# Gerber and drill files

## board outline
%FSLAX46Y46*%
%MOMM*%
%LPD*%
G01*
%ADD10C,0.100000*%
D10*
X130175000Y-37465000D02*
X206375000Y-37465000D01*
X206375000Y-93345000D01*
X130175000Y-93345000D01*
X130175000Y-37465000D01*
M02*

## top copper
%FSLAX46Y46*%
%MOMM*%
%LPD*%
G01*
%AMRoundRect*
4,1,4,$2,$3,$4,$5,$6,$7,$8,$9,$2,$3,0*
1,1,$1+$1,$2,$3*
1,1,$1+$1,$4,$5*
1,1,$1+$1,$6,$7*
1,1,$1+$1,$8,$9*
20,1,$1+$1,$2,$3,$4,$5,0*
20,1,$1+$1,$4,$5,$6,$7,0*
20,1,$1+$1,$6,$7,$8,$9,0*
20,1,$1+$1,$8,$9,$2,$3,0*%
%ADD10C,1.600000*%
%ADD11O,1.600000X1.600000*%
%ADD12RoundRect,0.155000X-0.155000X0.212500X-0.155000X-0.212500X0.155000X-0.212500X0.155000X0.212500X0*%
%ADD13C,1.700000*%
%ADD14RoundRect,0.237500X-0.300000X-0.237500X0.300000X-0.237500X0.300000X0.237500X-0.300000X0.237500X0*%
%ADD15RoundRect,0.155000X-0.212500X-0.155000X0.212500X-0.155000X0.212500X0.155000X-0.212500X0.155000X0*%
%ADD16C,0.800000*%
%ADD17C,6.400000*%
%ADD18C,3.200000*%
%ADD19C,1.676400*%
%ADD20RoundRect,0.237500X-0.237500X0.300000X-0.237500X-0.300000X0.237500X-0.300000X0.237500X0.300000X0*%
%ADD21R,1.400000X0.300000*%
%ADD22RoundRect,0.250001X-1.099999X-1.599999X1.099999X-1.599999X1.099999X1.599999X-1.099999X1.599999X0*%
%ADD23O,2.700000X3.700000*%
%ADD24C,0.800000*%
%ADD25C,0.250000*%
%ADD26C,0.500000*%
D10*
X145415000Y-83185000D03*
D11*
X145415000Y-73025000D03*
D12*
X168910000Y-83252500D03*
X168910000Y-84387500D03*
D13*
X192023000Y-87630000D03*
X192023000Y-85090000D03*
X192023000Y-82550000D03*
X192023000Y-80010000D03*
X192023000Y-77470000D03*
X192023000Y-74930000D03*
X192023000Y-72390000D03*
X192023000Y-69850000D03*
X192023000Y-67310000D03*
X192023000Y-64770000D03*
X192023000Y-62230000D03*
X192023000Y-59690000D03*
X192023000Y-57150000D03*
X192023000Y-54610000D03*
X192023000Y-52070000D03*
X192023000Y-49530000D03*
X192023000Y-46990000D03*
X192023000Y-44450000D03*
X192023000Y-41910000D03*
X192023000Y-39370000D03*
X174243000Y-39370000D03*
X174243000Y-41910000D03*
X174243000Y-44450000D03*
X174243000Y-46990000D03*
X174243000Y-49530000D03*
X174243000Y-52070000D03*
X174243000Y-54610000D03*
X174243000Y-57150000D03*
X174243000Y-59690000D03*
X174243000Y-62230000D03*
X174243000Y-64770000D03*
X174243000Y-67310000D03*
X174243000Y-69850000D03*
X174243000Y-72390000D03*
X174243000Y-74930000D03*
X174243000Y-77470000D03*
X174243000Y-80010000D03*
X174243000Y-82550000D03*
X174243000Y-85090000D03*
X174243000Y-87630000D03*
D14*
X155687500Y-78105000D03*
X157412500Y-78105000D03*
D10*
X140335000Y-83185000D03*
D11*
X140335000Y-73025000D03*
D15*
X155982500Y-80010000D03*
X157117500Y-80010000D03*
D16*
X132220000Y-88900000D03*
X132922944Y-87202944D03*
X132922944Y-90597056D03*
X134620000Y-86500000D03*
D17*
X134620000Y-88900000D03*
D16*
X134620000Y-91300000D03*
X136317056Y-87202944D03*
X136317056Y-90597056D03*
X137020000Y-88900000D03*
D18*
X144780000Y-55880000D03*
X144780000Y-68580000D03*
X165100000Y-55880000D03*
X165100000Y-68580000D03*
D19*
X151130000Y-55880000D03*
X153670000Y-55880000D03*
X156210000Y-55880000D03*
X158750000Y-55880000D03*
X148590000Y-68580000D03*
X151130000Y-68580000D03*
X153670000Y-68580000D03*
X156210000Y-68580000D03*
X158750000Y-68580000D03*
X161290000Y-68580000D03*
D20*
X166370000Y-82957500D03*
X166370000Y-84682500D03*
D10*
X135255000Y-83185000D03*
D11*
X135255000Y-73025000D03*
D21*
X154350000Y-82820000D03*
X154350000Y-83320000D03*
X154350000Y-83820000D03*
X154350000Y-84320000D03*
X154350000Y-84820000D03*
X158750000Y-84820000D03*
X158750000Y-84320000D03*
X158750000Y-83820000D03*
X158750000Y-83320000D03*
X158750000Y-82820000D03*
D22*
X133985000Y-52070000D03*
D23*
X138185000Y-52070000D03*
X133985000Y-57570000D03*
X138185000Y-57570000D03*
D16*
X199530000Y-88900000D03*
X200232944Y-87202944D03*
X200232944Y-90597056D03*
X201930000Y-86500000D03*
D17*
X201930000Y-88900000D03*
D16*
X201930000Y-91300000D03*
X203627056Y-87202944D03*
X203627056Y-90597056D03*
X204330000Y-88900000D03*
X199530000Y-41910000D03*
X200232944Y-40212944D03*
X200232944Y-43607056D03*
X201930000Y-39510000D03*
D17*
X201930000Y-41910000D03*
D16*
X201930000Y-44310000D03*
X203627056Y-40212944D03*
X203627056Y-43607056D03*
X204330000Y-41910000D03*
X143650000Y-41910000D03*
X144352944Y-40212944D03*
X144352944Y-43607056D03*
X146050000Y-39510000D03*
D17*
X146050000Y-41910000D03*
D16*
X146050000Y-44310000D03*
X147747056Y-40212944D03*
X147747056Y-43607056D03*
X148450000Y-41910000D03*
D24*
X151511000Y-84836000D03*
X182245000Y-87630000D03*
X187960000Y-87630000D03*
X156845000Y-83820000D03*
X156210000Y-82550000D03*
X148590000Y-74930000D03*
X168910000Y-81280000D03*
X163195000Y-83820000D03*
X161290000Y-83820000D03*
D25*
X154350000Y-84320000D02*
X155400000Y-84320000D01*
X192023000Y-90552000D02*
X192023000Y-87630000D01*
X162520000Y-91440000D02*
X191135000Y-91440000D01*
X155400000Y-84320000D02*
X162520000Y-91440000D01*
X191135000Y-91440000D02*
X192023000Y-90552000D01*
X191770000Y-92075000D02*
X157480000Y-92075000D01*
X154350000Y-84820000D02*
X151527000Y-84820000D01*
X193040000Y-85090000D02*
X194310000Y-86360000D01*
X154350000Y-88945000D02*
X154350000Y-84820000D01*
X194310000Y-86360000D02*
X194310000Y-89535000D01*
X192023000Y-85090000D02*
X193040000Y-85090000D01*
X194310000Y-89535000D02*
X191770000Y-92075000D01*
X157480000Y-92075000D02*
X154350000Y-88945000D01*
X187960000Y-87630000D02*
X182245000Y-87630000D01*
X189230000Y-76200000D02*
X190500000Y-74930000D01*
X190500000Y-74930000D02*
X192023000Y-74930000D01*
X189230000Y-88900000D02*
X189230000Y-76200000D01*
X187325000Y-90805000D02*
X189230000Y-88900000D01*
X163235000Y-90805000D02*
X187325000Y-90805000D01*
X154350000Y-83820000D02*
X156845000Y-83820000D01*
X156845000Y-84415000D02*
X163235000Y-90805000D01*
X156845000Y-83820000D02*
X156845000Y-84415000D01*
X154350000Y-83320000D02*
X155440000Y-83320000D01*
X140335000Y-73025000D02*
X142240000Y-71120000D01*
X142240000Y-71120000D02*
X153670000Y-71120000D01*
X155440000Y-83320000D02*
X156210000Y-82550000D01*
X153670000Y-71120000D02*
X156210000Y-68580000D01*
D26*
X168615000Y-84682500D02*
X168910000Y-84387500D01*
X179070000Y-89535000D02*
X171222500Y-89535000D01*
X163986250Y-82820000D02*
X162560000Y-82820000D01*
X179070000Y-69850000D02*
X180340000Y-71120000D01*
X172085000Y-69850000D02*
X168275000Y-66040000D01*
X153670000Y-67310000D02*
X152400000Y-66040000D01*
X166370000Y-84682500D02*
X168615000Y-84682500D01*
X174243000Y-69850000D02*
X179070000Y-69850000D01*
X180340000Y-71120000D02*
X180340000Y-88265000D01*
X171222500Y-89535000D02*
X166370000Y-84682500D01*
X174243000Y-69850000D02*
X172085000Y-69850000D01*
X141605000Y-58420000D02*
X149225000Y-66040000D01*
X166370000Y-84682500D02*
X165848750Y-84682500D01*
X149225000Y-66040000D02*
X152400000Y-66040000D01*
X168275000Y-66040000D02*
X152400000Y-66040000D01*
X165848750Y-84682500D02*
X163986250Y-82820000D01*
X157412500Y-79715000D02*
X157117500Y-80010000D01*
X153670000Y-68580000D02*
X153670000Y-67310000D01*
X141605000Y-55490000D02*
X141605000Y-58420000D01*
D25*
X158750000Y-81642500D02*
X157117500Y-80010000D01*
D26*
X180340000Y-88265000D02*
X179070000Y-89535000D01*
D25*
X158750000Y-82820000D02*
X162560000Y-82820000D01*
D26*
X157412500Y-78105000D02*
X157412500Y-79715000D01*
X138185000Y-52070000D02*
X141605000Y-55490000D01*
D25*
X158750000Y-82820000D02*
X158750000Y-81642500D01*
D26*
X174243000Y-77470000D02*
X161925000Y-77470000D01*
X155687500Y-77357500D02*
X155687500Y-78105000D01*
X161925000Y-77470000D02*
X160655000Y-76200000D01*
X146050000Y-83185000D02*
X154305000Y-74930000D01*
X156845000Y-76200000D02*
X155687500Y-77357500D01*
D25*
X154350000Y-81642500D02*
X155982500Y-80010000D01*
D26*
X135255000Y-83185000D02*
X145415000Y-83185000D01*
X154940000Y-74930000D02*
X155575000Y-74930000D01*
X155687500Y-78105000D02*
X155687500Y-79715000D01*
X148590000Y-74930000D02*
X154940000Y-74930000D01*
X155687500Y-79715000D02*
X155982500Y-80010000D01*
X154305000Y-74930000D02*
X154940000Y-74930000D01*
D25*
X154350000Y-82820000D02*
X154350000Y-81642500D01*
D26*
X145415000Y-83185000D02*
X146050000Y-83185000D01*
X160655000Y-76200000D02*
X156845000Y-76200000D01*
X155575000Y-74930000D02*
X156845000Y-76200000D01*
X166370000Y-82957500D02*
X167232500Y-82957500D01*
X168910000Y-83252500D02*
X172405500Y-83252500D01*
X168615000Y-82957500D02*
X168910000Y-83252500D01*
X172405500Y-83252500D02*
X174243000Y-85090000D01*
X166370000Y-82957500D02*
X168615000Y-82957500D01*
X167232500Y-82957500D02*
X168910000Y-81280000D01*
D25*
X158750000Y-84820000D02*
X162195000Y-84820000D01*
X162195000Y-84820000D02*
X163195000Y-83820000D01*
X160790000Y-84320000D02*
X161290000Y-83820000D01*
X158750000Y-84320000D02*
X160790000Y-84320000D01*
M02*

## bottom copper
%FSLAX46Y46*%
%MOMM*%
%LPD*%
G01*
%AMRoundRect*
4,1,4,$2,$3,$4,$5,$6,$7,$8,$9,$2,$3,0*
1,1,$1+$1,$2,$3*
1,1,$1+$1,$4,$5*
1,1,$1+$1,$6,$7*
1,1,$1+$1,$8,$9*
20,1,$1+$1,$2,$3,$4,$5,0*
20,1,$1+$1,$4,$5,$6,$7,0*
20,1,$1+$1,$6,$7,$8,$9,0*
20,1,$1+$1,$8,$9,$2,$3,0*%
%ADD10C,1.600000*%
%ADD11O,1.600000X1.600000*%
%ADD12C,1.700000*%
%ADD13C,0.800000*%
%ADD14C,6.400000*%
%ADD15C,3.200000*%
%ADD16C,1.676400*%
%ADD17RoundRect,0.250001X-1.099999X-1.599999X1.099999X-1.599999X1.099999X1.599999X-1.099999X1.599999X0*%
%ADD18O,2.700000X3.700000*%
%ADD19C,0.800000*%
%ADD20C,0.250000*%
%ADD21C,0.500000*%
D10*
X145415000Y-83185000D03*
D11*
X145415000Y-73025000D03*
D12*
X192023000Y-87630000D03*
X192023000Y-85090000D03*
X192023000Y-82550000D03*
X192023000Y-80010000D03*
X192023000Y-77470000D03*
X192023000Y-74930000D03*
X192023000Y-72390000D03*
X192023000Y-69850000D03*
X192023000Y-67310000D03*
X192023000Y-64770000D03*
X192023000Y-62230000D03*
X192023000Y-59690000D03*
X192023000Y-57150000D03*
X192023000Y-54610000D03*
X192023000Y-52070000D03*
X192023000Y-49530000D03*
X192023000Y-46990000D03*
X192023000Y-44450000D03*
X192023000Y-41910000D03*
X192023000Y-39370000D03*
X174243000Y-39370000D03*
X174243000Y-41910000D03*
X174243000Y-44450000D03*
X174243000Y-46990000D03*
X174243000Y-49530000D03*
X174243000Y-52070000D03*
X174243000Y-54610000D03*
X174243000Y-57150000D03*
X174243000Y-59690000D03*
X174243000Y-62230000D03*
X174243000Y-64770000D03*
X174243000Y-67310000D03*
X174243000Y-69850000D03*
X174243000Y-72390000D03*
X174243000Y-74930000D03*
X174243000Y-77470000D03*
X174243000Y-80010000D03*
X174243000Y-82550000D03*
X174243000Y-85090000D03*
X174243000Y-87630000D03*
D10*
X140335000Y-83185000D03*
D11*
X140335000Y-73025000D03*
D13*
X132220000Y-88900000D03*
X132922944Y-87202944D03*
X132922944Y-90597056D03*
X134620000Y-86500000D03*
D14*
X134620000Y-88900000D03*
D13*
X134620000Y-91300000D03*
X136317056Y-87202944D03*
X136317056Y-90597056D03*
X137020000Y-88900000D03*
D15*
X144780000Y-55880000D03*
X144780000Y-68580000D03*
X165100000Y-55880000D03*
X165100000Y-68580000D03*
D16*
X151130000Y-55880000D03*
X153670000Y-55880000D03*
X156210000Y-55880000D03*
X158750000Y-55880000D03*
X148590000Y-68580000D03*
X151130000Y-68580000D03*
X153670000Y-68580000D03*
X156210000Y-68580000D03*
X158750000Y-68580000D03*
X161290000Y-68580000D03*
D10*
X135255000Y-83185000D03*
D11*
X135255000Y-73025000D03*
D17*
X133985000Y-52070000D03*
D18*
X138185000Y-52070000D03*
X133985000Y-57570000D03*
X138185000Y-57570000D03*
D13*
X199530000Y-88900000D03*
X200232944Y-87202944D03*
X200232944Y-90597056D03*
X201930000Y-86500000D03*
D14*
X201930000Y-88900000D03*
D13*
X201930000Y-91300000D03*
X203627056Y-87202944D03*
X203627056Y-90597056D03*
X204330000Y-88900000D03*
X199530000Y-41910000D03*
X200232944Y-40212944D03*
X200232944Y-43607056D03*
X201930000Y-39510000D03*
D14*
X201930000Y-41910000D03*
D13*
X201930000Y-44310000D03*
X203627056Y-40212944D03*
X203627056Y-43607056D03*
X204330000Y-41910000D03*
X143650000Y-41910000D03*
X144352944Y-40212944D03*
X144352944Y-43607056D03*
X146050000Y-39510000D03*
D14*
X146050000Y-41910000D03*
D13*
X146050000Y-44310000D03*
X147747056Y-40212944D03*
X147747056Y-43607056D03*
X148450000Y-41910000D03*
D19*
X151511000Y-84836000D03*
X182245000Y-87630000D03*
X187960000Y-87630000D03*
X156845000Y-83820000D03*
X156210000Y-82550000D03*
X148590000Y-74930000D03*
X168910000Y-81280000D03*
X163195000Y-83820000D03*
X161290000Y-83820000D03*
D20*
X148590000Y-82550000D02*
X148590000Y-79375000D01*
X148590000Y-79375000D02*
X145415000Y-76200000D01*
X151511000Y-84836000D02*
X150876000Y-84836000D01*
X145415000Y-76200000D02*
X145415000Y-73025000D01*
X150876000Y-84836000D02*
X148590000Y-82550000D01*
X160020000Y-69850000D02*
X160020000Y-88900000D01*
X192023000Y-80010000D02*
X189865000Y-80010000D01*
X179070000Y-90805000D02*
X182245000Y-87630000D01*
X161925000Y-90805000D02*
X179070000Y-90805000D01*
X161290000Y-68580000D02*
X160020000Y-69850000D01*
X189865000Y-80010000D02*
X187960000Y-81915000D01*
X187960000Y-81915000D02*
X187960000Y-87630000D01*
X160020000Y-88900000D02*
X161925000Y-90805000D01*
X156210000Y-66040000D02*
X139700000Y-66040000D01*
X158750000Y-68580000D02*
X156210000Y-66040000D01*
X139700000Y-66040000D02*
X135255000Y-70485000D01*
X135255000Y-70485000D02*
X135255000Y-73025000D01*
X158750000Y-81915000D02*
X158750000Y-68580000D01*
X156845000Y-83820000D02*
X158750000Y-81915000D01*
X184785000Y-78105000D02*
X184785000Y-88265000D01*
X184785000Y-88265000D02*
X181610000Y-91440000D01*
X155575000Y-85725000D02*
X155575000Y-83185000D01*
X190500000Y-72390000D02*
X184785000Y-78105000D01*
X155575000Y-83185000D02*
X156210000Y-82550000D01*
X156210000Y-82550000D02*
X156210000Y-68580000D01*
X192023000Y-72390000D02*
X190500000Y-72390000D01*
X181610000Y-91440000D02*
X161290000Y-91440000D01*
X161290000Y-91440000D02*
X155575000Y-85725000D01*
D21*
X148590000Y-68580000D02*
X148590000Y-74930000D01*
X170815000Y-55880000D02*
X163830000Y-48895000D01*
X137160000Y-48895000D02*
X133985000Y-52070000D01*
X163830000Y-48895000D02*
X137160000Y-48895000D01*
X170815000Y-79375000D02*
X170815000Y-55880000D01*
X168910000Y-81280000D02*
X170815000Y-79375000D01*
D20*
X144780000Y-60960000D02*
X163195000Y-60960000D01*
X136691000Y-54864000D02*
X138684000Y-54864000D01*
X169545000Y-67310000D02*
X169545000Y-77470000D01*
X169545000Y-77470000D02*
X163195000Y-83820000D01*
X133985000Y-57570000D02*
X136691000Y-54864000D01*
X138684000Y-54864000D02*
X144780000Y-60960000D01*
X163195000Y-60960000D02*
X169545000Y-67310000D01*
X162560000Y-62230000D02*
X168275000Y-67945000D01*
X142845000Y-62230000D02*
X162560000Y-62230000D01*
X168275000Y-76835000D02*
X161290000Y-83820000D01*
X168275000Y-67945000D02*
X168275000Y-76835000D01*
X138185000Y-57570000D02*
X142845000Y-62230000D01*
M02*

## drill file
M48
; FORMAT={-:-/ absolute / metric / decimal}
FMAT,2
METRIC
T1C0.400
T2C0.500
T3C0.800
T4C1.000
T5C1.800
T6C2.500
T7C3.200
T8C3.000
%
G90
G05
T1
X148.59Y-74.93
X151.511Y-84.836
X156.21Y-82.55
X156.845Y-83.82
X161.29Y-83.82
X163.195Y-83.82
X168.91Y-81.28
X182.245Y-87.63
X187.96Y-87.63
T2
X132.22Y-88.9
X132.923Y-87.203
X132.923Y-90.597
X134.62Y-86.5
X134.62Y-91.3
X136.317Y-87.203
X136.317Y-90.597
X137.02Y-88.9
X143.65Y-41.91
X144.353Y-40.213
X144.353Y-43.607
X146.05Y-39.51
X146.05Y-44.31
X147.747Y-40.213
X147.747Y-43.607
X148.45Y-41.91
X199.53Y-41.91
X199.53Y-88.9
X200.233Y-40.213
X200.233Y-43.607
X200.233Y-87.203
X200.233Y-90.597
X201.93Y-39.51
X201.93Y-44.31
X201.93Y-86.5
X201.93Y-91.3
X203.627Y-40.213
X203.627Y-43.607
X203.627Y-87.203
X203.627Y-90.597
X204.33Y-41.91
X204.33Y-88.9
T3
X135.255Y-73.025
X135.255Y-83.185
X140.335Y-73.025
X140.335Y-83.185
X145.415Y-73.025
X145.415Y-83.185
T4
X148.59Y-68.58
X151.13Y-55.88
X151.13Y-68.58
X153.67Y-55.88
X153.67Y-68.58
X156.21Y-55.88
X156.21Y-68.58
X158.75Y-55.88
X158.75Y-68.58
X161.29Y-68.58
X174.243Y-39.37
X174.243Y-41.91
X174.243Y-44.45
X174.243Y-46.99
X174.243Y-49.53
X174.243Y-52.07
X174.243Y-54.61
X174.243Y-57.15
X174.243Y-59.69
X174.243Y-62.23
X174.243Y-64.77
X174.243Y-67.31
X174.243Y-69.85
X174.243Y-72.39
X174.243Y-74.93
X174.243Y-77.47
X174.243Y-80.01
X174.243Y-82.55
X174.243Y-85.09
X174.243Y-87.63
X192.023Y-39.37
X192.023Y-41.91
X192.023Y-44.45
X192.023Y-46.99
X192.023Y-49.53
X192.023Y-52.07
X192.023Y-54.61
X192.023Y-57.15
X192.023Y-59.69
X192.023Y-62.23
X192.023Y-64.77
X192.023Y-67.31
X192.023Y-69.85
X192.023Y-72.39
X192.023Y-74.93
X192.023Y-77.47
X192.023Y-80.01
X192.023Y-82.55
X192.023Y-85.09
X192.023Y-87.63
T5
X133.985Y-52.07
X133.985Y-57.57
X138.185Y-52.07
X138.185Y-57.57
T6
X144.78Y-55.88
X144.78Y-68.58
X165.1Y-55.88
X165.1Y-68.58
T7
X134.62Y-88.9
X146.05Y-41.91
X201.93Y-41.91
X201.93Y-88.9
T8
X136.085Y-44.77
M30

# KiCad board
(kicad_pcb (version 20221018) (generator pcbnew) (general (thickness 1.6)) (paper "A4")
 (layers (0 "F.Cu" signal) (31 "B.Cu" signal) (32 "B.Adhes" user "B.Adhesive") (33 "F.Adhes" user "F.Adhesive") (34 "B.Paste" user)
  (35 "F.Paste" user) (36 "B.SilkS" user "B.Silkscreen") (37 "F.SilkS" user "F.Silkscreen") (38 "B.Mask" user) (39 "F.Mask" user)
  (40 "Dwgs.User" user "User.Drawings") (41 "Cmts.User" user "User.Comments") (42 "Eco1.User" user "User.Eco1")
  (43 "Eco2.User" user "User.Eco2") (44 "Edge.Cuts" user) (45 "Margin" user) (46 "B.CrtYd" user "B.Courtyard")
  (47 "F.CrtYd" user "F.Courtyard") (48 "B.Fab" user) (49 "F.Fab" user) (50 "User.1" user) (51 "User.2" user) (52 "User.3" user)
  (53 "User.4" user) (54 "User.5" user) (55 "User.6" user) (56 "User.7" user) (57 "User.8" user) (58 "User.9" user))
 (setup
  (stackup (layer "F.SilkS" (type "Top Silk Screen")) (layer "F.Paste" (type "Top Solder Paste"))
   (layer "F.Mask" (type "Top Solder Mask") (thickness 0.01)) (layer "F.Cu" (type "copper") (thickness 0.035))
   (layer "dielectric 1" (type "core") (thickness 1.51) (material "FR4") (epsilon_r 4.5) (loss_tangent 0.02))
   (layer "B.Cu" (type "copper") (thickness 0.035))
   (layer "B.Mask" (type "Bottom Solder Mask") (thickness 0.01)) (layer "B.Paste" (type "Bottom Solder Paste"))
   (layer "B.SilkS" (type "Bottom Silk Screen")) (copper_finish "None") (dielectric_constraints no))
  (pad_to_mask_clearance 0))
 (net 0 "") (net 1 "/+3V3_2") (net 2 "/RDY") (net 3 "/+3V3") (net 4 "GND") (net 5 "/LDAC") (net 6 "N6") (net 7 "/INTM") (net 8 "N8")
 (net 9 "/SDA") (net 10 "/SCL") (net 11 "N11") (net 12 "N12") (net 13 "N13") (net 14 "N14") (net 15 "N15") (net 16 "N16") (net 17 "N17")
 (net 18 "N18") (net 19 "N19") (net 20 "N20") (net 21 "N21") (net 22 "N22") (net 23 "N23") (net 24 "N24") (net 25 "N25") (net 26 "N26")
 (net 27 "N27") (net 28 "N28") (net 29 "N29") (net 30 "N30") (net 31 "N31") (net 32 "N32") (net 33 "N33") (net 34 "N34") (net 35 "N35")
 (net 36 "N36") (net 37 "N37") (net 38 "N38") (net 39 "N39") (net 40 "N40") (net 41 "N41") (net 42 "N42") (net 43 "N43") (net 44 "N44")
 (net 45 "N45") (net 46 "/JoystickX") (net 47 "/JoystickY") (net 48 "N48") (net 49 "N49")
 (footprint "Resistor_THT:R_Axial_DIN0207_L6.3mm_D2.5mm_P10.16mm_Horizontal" (layer "F.Cu") (at 145.415 83.185 90)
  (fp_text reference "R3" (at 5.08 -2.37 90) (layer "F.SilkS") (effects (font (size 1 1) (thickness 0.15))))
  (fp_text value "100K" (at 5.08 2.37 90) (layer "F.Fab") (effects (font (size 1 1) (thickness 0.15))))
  (pad "1" thru_hole circle (at 0 0 90) (size 1.6 1.6) (drill 0.8) (layers "*.Cu" "*.Mask") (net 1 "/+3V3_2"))
  (pad "2" thru_hole oval (at 10.16 0 90) (size 1.6 1.6) (drill 0.8) (layers "*.Cu" "*.Mask") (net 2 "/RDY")))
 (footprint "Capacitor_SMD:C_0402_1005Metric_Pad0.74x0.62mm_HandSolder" (layer "F.Cu") (at 168.91 83.82 -90)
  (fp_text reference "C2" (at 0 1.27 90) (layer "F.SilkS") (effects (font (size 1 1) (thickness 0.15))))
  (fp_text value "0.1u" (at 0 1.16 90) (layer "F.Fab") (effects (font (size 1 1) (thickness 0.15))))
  (pad "1" smd roundrect (at -0.5675 0 270) (size 0.735 0.62) (layers "F.Cu" "F.Paste" "F.Mask") (roundrect_rratio 0.25) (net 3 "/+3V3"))
  (pad "2" smd roundrect (at 0.5675 0 270) (size 0.735 0.62) (layers "F.Cu" "F.Paste" "F.Mask") (roundrect_rratio 0.25) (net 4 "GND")))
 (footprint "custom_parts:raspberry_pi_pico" (layer "F.Cu") (at 183.515 64.712 90)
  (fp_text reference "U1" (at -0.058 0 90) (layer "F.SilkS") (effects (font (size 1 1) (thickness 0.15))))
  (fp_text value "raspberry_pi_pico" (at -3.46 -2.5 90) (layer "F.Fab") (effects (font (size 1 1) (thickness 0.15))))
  (pad "1" thru_hole circle (at -22.918 8.508) (size 1.7 1.7) (drill 1) (layers "*.Cu" "*.Mask") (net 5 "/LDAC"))
  (pad "2" thru_hole circle (at -20.378 8.508) (size 1.7 1.7) (drill 1) (layers "*.Cu" "*.Mask") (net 2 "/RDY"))
  (pad "3" thru_hole circle (at -17.838 8.508) (size 1.7 1.7) (drill 1) (layers "*.Cu" "*.Mask") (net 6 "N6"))
  (pad "4" thru_hole circle (at -15.298 8.508) (size 1.7 1.7) (drill 1) (layers "*.Cu" "*.Mask") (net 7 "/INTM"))
  (pad "5" thru_hole circle (at -12.758 8.508) (size 1.7 1.7) (drill 1) (layers "*.Cu" "*.Mask") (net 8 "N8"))
  (pad "6" thru_hole circle (at -10.218 8.508) (size 1.7 1.7) (drill 1) (layers "*.Cu" "*.Mask") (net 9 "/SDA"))
  (pad "7" thru_hole circle (at -7.678 8.508) (size 1.7 1.7) (drill 1) (layers "*.Cu" "*.Mask") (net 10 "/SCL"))
  (pad "8" thru_hole circle (at -5.138 8.508) (size 1.7 1.7) (drill 1) (layers "*.Cu" "*.Mask") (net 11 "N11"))
  (pad "9" thru_hole circle (at -2.598 8.508) (size 1.7 1.7) (drill 1) (layers "*.Cu" "*.Mask") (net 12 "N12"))
  (pad "10" thru_hole circle (at -0.058 8.508) (size 1.7 1.7) (drill 1) (layers "*.Cu" "*.Mask") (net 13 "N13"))
  (pad "11" thru_hole circle (at 2.482 8.508) (size 1.7 1.7) (drill 1) (layers "*.Cu" "*.Mask") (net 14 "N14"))
  (pad "12" thru_hole circle (at 5.022 8.508) (size 1.7 1.7) (drill 1) (layers "*.Cu" "*.Mask") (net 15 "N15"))
  (pad "13" thru_hole circle (at 7.562 8.508) (size 1.7 1.7) (drill 1) (layers "*.Cu" "*.Mask") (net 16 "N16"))
  (pad "14" thru_hole circle (at 10.102 8.508) (size 1.7 1.7) (drill 1) (layers "*.Cu" "*.Mask") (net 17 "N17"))
  (pad "15" thru_hole circle (at 12.642 8.508) (size 1.7 1.7) (drill 1) (layers "*.Cu" "*.Mask") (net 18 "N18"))
  (pad "16" thru_hole circle (at 15.182 8.508) (size 1.7 1.7) (drill 1) (layers "*.Cu" "*.Mask") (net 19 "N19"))
  (pad "17" thru_hole circle (at 17.722 8.508) (size 1.7 1.7) (drill 1) (layers "*.Cu" "*.Mask") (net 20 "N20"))
  (pad "18" thru_hole circle (at 20.262 8.508) (size 1.7 1.7) (drill 1) (layers "*.Cu" "*.Mask") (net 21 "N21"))
  (pad "19" thru_hole circle (at 22.802 8.508) (size 1.7 1.7) (drill 1) (layers "*.Cu" "*.Mask") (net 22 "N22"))
  (pad "20" thru_hole circle (at 25.342 8.508) (size 1.7 1.7) (drill 1) (layers "*.Cu" "*.Mask") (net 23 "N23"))
  (pad "21" thru_hole circle (at 25.342 -9.272) (size 1.7 1.7) (drill 1) (layers "*.Cu" "*.Mask") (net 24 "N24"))
  (pad "22" thru_hole circle (at 22.802 -9.272) (size 1.7 1.7) (drill 1) (layers "*.Cu" "*.Mask") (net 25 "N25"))
  (pad "23" thru_hole circle (at 20.262 -9.272) (size 1.7 1.7) (drill 1) (layers "*.Cu" "*.Mask") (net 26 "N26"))
  (pad "24" thru_hole circle (at 17.722 -9.272) (size 1.7 1.7) (drill 1) (layers "*.Cu" "*.Mask") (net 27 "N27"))
  (pad "25" thru_hole circle (at 15.182 -9.272) (size 1.7 1.7) (drill 1) (layers "*.Cu" "*.Mask") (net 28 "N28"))
  (pad "26" thru_hole circle (at 12.642 -9.272) (size 1.7 1.7) (drill 1) (layers "*.Cu" "*.Mask") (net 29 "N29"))
  (pad "27" thru_hole circle (at 10.102 -9.272) (size 1.7 1.7) (drill 1) (layers "*.Cu" "*.Mask") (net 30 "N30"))
  (pad "28" thru_hole circle (at 7.562 -9.272) (size 1.7 1.7) (drill 1) (layers "*.Cu" "*.Mask") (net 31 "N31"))
  (pad "29" thru_hole circle (at 5.022 -9.272) (size 1.7 1.7) (drill 1) (layers "*.Cu" "*.Mask") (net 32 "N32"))
  (pad "30" thru_hole circle (at 2.482 -9.272) (size 1.7 1.7) (drill 1) (layers "*.Cu" "*.Mask") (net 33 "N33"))
  (pad "31" thru_hole circle (at -0.058 -9.272) (size 1.7 1.7) (drill 1) (layers "*.Cu" "*.Mask") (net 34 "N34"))
  (pad "32" thru_hole circle (at -2.598 -9.272) (size 1.7 1.7) (drill 1) (layers "*.Cu" "*.Mask") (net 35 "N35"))
  (pad "33" thru_hole circle (at -5.138 -9.272) (size 1.7 1.7) (drill 1) (layers "*.Cu" "*.Mask") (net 4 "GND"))
  (pad "34" thru_hole circle (at -7.678 -9.272) (size 1.7 1.7) (drill 1) (layers "*.Cu" "*.Mask") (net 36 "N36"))
  (pad "35" thru_hole circle (at -10.218 -9.272) (size 1.7 1.7) (drill 1) (layers "*.Cu" "*.Mask") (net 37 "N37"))
  (pad "36" thru_hole circle (at -12.758 -9.272) (size 1.7 1.7) (drill 1) (layers "*.Cu" "*.Mask") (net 1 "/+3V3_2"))
  (pad "37" thru_hole circle (at -15.298 -9.272) (size 1.7 1.7) (drill 1) (layers "*.Cu" "*.Mask") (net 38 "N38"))
  (pad "38" thru_hole circle (at -17.838 -9.272) (size 1.7 1.7) (drill 1) (layers "*.Cu" "*.Mask") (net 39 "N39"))
  (pad "39" thru_hole circle (at -20.378 -9.272) (size 1.7 1.7) (drill 1) (layers "*.Cu" "*.Mask") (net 3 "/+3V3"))
  (pad "40" thru_hole circle (at -22.918 -9.272) (size 1.7 1.7) (drill 1) (layers "*.Cu" "*.Mask") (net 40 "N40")))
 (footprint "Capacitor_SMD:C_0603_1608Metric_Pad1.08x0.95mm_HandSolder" (layer "F.Cu") (at 156.55 78.105)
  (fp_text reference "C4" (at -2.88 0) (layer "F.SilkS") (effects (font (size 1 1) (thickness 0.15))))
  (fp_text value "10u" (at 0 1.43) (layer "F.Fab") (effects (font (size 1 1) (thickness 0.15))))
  (pad "1" smd roundrect (at -0.8625 0) (size 1.075 0.95) (layers "F.Cu" "F.Paste" "F.Mask") (roundrect_rratio 0.25) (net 1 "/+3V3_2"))
  (pad "2" smd roundrect (at 0.8625 0) (size 1.075 0.95) (layers "F.Cu" "F.Paste" "F.Mask") (roundrect_rratio 0.25) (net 4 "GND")))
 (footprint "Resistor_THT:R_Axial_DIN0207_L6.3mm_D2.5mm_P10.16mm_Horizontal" (layer "F.Cu") (at 140.335 83.185 90)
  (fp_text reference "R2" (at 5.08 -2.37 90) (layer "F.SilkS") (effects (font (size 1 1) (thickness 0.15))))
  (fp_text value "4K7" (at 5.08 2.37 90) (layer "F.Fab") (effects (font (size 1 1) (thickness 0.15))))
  (pad "1" thru_hole circle (at 0 0 90) (size 1.6 1.6) (drill 0.8) (layers "*.Cu" "*.Mask") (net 1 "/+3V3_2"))
  (pad "2" thru_hole oval (at 10.16 0 90) (size 1.6 1.6) (drill 0.8) (layers "*.Cu" "*.Mask") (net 10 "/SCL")))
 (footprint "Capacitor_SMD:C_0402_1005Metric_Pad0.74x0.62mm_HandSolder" (layer "F.Cu") (at 156.55 80.01)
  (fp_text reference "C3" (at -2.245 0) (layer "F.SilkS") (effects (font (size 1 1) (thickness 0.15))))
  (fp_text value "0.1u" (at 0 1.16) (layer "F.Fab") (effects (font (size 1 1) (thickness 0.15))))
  (pad "1" smd roundrect (at -0.5675 0) (size 0.735 0.62) (layers "F.Cu" "F.Paste" "F.Mask") (roundrect_rratio 0.25) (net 1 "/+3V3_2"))
  (pad "2" smd roundrect (at 0.5675 0) (size 0.735 0.62) (layers "F.Cu" "F.Paste" "F.Mask") (roundrect_rratio 0.25) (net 4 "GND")))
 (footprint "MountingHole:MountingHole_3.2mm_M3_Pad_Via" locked (layer "F.Cu") (at 134.62 88.9)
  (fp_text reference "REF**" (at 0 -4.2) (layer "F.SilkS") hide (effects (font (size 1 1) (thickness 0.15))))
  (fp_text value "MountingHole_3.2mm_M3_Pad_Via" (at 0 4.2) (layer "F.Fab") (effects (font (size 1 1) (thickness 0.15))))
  (pad "1" thru_hole circle locked (at -2.4 0) (size 0.8 0.8) (drill 0.5) (layers "*.Cu" "*.Mask"))
  (pad "1" thru_hole circle locked (at -1.697056 -1.697056) (size 0.8 0.8) (drill 0.5) (layers "*.Cu" "*.Mask"))
  (pad "1" thru_hole circle locked (at -1.697056 1.697056) (size 0.8 0.8) (drill 0.5) (layers "*.Cu" "*.Mask"))
  (pad "1" thru_hole circle locked (at 0 -2.4) (size 0.8 0.8) (drill 0.5) (layers "*.Cu" "*.Mask"))
  (pad "1" thru_hole circle locked (at 0 0) (size 6.4 6.4) (drill 3.2) (layers "*.Cu" "*.Mask"))
  (pad "1" thru_hole circle locked (at 0 2.4) (size 0.8 0.8) (drill 0.5) (layers "*.Cu" "*.Mask"))
  (pad "1" thru_hole circle locked (at 1.697056 -1.697056) (size 0.8 0.8) (drill 0.5) (layers "*.Cu" "*.Mask"))
  (pad "1" thru_hole circle locked (at 1.697056 1.697056) (size 0.8 0.8) (drill 0.5) (layers "*.Cu" "*.Mask"))
  (pad "1" thru_hole circle locked (at 2.4 0) (size 0.8 0.8) (drill 0.5) (layers "*.Cu" "*.Mask")))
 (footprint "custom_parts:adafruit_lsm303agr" (layer "F.Cu") (at 154.94 63.5)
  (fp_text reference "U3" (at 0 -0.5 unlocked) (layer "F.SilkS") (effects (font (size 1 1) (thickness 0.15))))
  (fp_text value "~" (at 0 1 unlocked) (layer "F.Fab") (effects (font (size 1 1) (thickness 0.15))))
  (pad "" thru_hole circle (at -10.16 -7.62) (size 3.2 3.2) (drill 2.5) (layers "*.Cu" "*.Mask") (zone_connect 0))
  (pad "" thru_hole circle (at -10.16 5.08) (size 3.2 3.2) (drill 2.5) (layers "*.Cu" "*.Mask") (zone_connect 0))
  (pad "" thru_hole circle (at 10.16 -7.62) (size 3.2 3.2) (drill 2.5) (layers "*.Cu" "*.Mask") (zone_connect 0))
  (pad "" thru_hole circle (at 10.16 5.08) (size 3.2 3.2) (drill 2.5) (layers "*.Cu" "*.Mask") (zone_connect 0))
  (pad "0" thru_hole circle (at -3.81 -7.62 90) (size 1.6764 1.6764) (drill 1) (layers "*.Cu" "*.Mask") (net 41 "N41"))
  (pad "1" thru_hole circle (at -1.27 -7.62 90) (size 1.6764 1.6764) (drill 1) (layers "*.Cu" "*.Mask") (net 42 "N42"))
  (pad "2" thru_hole circle (at 1.27 -7.62 90) (size 1.6764 1.6764) (drill 1) (layers "*.Cu" "*.Mask") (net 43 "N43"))
  (pad "3" thru_hole circle (at 3.81 -7.62 90) (size 1.6764 1.6764) (drill 1) (layers "*.Cu" "*.Mask") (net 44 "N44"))
  (pad "4" thru_hole circle (at -6.35 5.08 90) (size 1.6764 1.6764) (drill 1) (layers "*.Cu" "*.Mask") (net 1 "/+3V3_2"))
  (pad "5" thru_hole circle (at -3.81 5.08 90) (size 1.6764 1.6764) (drill 1) (layers "*.Cu" "*.Mask") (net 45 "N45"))
  (pad "6" thru_hole circle (at -1.27 5.08 90) (size 1.6764 1.6764) (drill 1) (layers "*.Cu" "*.Mask") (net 4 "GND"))
  (pad "7" thru_hole circle (at 1.27 5.08 90) (size 1.6764 1.6764) (drill 1) (layers "*.Cu" "*.Mask") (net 10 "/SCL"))
  (pad "8" thru_hole circle (at 3.81 5.08 90) (size 1.6764 1.6764) (drill 1) (layers "*.Cu" "*.Mask") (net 9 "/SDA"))
  (pad "9" thru_hole circle (at 6.35 5.08 90) (size 1.6764 1.6764) (drill 1) (layers "*.Cu" "*.Mask") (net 7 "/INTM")))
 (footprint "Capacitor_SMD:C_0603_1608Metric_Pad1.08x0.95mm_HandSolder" (layer "F.Cu") (at 166.37 83.82 -90)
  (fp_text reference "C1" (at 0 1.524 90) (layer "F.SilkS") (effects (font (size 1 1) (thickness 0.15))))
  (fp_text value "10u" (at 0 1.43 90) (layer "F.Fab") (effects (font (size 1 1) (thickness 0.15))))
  (pad "1" smd roundrect (at -0.8625 0 270) (size 1.075 0.95) (layers "F.Cu" "F.Paste" "F.Mask") (roundrect_rratio 0.25) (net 3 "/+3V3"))
  (pad "2" smd roundrect (at 0.8625 0 270) (size 1.075 0.95) (layers "F.Cu" "F.Paste" "F.Mask") (roundrect_rratio 0.25) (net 4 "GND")))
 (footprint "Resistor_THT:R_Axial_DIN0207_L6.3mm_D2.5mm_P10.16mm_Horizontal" (layer "F.Cu") (at 135.255 83.185 90)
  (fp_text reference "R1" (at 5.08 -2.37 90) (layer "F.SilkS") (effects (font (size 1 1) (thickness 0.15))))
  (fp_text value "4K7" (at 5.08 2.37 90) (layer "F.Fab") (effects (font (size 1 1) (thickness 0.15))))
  (pad "1" thru_hole circle (at 0 0 90) (size 1.6 1.6) (drill 0.8) (layers "*.Cu" "*.Mask") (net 1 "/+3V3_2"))
  (pad "2" thru_hole oval (at 10.16 0 90) (size 1.6 1.6) (drill 0.8) (layers "*.Cu" "*.Mask") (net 9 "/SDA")))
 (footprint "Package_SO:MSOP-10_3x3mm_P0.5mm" (layer "F.Cu") (at 156.55 83.82)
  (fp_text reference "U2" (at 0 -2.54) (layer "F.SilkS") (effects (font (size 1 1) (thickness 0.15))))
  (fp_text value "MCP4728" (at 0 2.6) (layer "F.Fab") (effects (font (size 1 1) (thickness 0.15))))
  (pad "1" smd rect (at -2.2 -1) (size 1.4 0.3) (layers "F.Cu" "F.Paste" "F.Mask") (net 1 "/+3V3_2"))
  (pad "2" smd rect (at -2.2 -0.5) (size 1.4 0.3) (layers "F.Cu" "F.Paste" "F.Mask") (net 10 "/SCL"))
  (pad "3" smd rect (at -2.2 0) (size 1.4 0.3) (layers "F.Cu" "F.Paste" "F.Mask") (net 9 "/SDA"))
  (pad "4" smd rect (at -2.2 0.5) (size 1.4 0.3) (layers "F.Cu" "F.Paste" "F.Mask") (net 5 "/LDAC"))
  (pad "5" smd rect (at -2.2 1) (size 1.4 0.3) (layers "F.Cu" "F.Paste" "F.Mask") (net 2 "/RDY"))
  (pad "6" smd rect (at 2.2 1) (size 1.4 0.3) (layers "F.Cu" "F.Paste" "F.Mask") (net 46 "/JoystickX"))
  (pad "7" smd rect (at 2.2 0.5) (size 1.4 0.3) (layers "F.Cu" "F.Paste" "F.Mask") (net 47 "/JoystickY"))
  (pad "8" smd rect (at 2.2 0) (size 1.4 0.3) (layers "F.Cu" "F.Paste" "F.Mask") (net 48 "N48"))
  (pad "9" smd rect (at 2.2 -0.5) (size 1.4 0.3) (layers "F.Cu" "F.Paste" "F.Mask") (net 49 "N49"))
  (pad "10" smd rect (at 2.2 -1) (size 1.4 0.3) (layers "F.Cu" "F.Paste" "F.Mask") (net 4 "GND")))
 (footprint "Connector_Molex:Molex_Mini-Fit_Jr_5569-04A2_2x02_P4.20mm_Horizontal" (layer "F.Cu") (at 133.985 52.07)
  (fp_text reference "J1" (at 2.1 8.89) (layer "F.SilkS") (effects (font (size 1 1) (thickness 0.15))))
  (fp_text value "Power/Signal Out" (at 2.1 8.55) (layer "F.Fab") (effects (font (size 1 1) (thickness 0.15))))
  (pad "" np_thru_hole circle (at 2.1 -7.3) (size 3 3) (drill 3) (layers "*.Cu" "*.Mask"))
  (pad "1" thru_hole roundrect (at 0 0) (size 2.7 3.7) (drill 1.8) (layers "*.Cu" "*.Mask") (roundrect_rratio 0.09259296296) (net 3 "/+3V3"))
  (pad "2" thru_hole oval (at 4.2 0) (size 2.7 3.7) (drill 1.8) (layers "*.Cu" "*.Mask") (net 4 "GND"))
  (pad "3" thru_hole oval (at 0 5.5) (size 2.7 3.7) (drill 1.8) (layers "*.Cu" "*.Mask") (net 46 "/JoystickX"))
  (pad "4" thru_hole oval (at 4.2 5.5) (size 2.7 3.7) (drill 1.8) (layers "*.Cu" "*.Mask") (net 47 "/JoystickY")))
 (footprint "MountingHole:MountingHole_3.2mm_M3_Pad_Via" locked (layer "F.Cu") (at 201.93 88.9)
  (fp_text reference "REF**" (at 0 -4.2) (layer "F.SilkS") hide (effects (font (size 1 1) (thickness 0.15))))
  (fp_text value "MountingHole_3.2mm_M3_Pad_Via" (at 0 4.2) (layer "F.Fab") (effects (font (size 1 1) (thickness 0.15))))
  (pad "1" thru_hole circle locked (at -2.4 0) (size 0.8 0.8) (drill 0.5) (layers "*.Cu" "*.Mask"))
  (pad "1" thru_hole circle locked (at -1.697056 -1.697056) (size 0.8 0.8) (drill 0.5) (layers "*.Cu" "*.Mask"))
  (pad "1" thru_hole circle locked (at -1.697056 1.697056) (size 0.8 0.8) (drill 0.5) (layers "*.Cu" "*.Mask"))
  (pad "1" thru_hole circle locked (at 0 -2.4) (size 0.8 0.8) (drill 0.5) (layers "*.Cu" "*.Mask"))
  (pad "1" thru_hole circle locked (at 0 0) (size 6.4 6.4) (drill 3.2) (layers "*.Cu" "*.Mask"))
  (pad "1" thru_hole circle locked (at 0 2.4) (size 0.8 0.8) (drill 0.5) (layers "*.Cu" "*.Mask"))
  (pad "1" thru_hole circle locked (at 1.697056 -1.697056) (size 0.8 0.8) (drill 0.5) (layers "*.Cu" "*.Mask"))
  (pad "1" thru_hole circle locked (at 1.697056 1.697056) (size 0.8 0.8) (drill 0.5) (layers "*.Cu" "*.Mask"))
  (pad "1" thru_hole circle locked (at 2.4 0) (size 0.8 0.8) (drill 0.5) (layers "*.Cu" "*.Mask")))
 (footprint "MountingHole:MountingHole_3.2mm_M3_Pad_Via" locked (layer "F.Cu") (at 201.93 41.91)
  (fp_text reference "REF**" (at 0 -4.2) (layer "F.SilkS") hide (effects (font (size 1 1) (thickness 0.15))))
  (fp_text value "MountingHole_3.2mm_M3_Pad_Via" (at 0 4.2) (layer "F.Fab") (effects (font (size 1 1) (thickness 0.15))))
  (pad "1" thru_hole circle locked (at -2.4 0) (size 0.8 0.8) (drill 0.5) (layers "*.Cu" "*.Mask"))
  (pad "1" thru_hole circle locked (at -1.697056 -1.697056) (size 0.8 0.8) (drill 0.5) (layers "*.Cu" "*.Mask"))
  (pad "1" thru_hole circle locked (at -1.697056 1.697056) (size 0.8 0.8) (drill 0.5) (layers "*.Cu" "*.Mask"))
  (pad "1" thru_hole circle locked (at 0 -2.4) (size 0.8 0.8) (drill 0.5) (layers "*.Cu" "*.Mask"))
  (pad "1" thru_hole circle locked (at 0 0) (size 6.4 6.4) (drill 3.2) (layers "*.Cu" "*.Mask"))
  (pad "1" thru_hole circle locked (at 0 2.4) (size 0.8 0.8) (drill 0.5) (layers "*.Cu" "*.Mask"))
  (pad "1" thru_hole circle locked (at 1.697056 -1.697056) (size 0.8 0.8) (drill 0.5) (layers "*.Cu" "*.Mask"))
  (pad "1" thru_hole circle locked (at 1.697056 1.697056) (size 0.8 0.8) (drill 0.5) (layers "*.Cu" "*.Mask"))
  (pad "1" thru_hole circle locked (at 2.4 0) (size 0.8 0.8) (drill 0.5) (layers "*.Cu" "*.Mask")))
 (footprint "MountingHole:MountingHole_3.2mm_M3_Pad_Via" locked (layer "F.Cu") (at 146.05 41.91)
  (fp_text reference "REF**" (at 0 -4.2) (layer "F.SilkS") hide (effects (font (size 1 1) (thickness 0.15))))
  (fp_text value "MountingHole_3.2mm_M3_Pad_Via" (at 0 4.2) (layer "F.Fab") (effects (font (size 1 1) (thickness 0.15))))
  (pad "1" thru_hole circle locked (at -2.4 0) (size 0.8 0.8) (drill 0.5) (layers "*.Cu" "*.Mask"))
  (pad "1" thru_hole circle locked (at -1.697056 -1.697056) (size 0.8 0.8) (drill 0.5) (layers "*.Cu" "*.Mask"))
  (pad "1" thru_hole circle locked (at -1.697056 1.697056) (size 0.8 0.8) (drill 0.5) (layers "*.Cu" "*.Mask"))
  (pad "1" thru_hole circle locked (at 0 -2.4) (size 0.8 0.8) (drill 0.5) (layers "*.Cu" "*.Mask"))
  (pad "1" thru_hole circle locked (at 0 0) (size 6.4 6.4) (drill 3.2) (layers "*.Cu" "*.Mask"))
  (pad "1" thru_hole circle locked (at 0 2.4) (size 0.8 0.8) (drill 0.5) (layers "*.Cu" "*.Mask"))
  (pad "1" thru_hole circle locked (at 1.697056 -1.697056) (size 0.8 0.8) (drill 0.5) (layers "*.Cu" "*.Mask"))
  (pad "1" thru_hole circle locked (at 1.697056 1.697056) (size 0.8 0.8) (drill 0.5) (layers "*.Cu" "*.Mask"))
  (pad "1" thru_hole circle locked (at 2.4 0) (size 0.8 0.8) (drill 0.5) (layers "*.Cu" "*.Mask")))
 (gr_rect (start 130.175 37.465) (end 206.375 93.345) (stroke (width 0.1) (type default)) (fill none) (layer "Edge.Cuts"))
 (segment (start 154.35 84.32) (end 155.4 84.32) (width 0.25) (layer "F.Cu") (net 5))
 (segment (start 192.023 90.552) (end 192.023 87.63) (width 0.25) (layer "F.Cu") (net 5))
 (segment (start 162.52 91.44) (end 191.135 91.44) (width 0.25) (layer "F.Cu") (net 5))
 (segment (start 155.4 84.32) (end 162.52 91.44) (width 0.25) (layer "F.Cu") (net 5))
 (segment (start 191.135 91.44) (end 192.023 90.552) (width 0.25) (layer "F.Cu") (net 5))
 (segment (start 191.77 92.075) (end 157.48 92.075) (width 0.25) (layer "F.Cu") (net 2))
 (segment (start 154.35 84.82) (end 151.527 84.82) (width 0.25) (layer "F.Cu") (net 2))
 (segment (start 193.04 85.09) (end 194.31 86.36) (width 0.25) (layer "F.Cu") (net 2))
 (segment (start 154.35 88.945) (end 154.35 84.82) (width 0.25) (layer "F.Cu") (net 2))
 (segment (start 194.31 86.36) (end 194.31 89.535) (width 0.25) (layer "F.Cu") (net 2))
 (segment (start 192.023 85.09) (end 193.04 85.09) (width 0.25) (layer "F.Cu") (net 2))
 (segment (start 194.31 89.535) (end 191.77 92.075) (width 0.25) (layer "F.Cu") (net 2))
 (segment (start 157.48 92.075) (end 154.35 88.945) (width 0.25) (layer "F.Cu") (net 2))
 (via (at 151.511 84.836) (size 0.8) (drill 0.4) (layers "F.Cu" "B.Cu") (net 2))
 (segment (start 148.59 82.55) (end 148.59 79.375) (width 0.25) (layer "B.Cu") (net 2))
 (segment (start 148.59 79.375) (end 145.415 76.2) (width 0.25) (layer "B.Cu") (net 2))
 (segment (start 151.511 84.836) (end 150.876 84.836) (width 0.25) (layer "B.Cu") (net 2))
 (segment (start 145.415 76.2) (end 145.415 73.025) (width 0.25) (layer "B.Cu") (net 2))
 (segment (start 150.876 84.836) (end 148.59 82.55) (width 0.25) (layer "B.Cu") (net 2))
 (segment (start 187.96 87.63) (end 182.245 87.63) (width 0.25) (layer "F.Cu") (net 7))
 (via (at 182.245 87.63) (size 0.8) (drill 0.4) (layers "F.Cu" "B.Cu") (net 7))
 (via (at 187.96 87.63) (size 0.8) (drill 0.4) (layers "F.Cu" "B.Cu") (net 7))
 (segment (start 160.02 69.85) (end 160.02 88.9) (width 0.25) (layer "B.Cu") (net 7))
 (segment (start 192.023 80.01) (end 189.865 80.01) (width 0.25) (layer "B.Cu") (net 7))
 (segment (start 179.07 90.805) (end 182.245 87.63) (width 0.25) (layer "B.Cu") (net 7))
 (segment (start 161.925 90.805) (end 179.07 90.805) (width 0.25) (layer "B.Cu") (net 7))
 (segment (start 161.29 68.58) (end 160.02 69.85) (width 0.25) (layer "B.Cu") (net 7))
 (segment (start 189.865 80.01) (end 187.96 81.915) (width 0.25) (layer "B.Cu") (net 7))
 (segment (start 187.96 81.915) (end 187.96 87.63) (width 0.25) (layer "B.Cu") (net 7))
 (segment (start 160.02 88.9) (end 161.925 90.805) (width 0.25) (layer "B.Cu") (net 7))
 (segment (start 189.23 76.2) (end 190.5 74.93) (width 0.25) (layer "F.Cu") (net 9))
 (segment (start 190.5 74.93) (end 192.023 74.93) (width 0.25) (layer "F.Cu") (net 9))
 (segment (start 189.23 88.9) (end 189.23 76.2) (width 0.25) (layer "F.Cu") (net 9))
 (segment (start 187.325 90.805) (end 189.23 88.9) (width 0.25) (layer "F.Cu") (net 9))
 (segment (start 163.235 90.805) (end 187.325 90.805) (width 0.25) (layer "F.Cu") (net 9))
 (segment (start 154.35 83.82) (end 156.845 83.82) (width 0.25) (layer "F.Cu") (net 9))
 (segment (start 156.845 84.415) (end 163.235 90.805) (width 0.25) (layer "F.Cu") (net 9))
 (segment (start 156.845 83.82) (end 156.845 84.415) (width 0.25) (layer "F.Cu") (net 9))
 (via (at 156.845 83.82) (size 0.8) (drill 0.4) (layers "F.Cu" "B.Cu") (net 9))
 (segment (start 156.21 66.04) (end 139.7 66.04) (width 0.25) (layer "B.Cu") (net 9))
 (segment (start 158.75 68.58) (end 156.21 66.04) (width 0.25) (layer "B.Cu") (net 9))
 (segment (start 139.7 66.04) (end 135.255 70.485) (width 0.25) (layer "B.Cu") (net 9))
 (segment (start 135.255 70.485) (end 135.255 73.025) (width 0.25) (layer "B.Cu") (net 9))
 (segment (start 158.75 81.915) (end 158.75 68.58) (width 0.25) (layer "B.Cu") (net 9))
 (segment (start 156.845 83.82) (end 158.75 81.915) (width 0.25) (layer "B.Cu") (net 9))
 (segment (start 154.35 83.32) (end 155.44 83.32) (width 0.25) (layer "F.Cu") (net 10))
 (segment (start 140.335 73.025) (end 142.24 71.12) (width 0.25) (layer "F.Cu") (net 10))
 (segment (start 142.24 71.12) (end 153.67 71.12) (width 0.25) (layer "F.Cu") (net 10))
 (segment (start 155.44 83.32) (end 156.21 82.55) (width 0.25) (layer "F.Cu") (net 10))
 (segment (start 153.67 71.12) (end 156.21 68.58) (width 0.25) (layer "F.Cu") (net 10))
 (via (at 156.21 82.55) (size 0.8) (drill 0.4) (layers "F.Cu" "B.Cu") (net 10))
 (segment (start 184.785 78.105) (end 184.785 88.265) (width 0.25) (layer "B.Cu") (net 10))
 (segment (start 184.785 88.265) (end 181.61 91.44) (width 0.25) (layer "B.Cu") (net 10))
 (segment (start 155.575 85.725) (end 155.575 83.185) (width 0.25) (layer "B.Cu") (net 10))
 (segment (start 190.5 72.39) (end 184.785 78.105) (width 0.25) (layer "B.Cu") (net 10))
 (segment (start 155.575 83.185) (end 156.21 82.55) (width 0.25) (layer "B.Cu") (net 10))
 (segment (start 156.21 82.55) (end 156.21 68.58) (width 0.25) (layer "B.Cu") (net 10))
 (segment (start 192.023 72.39) (end 190.5 72.39) (width 0.25) (layer "B.Cu") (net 10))
 (segment (start 181.61 91.44) (end 161.29 91.44) (width 0.25) (layer "B.Cu") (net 10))
 (segment (start 161.29 91.44) (end 155.575 85.725) (width 0.25) (layer "B.Cu") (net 10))
 (segment (start 168.615 84.6825) (end 168.91 84.3875) (width 0.5) (layer "F.Cu") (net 4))
 (segment (start 179.07 89.535) (end 171.2225 89.535) (width 0.5) (layer "F.Cu") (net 4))
 (segment (start 163.98625 82.82) (end 162.56 82.82) (width 0.5) (layer "F.Cu") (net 4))
 (segment (start 179.07 69.85) (end 180.34 71.12) (width 0.5) (layer "F.Cu") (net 4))
 (segment (start 172.085 69.85) (end 168.275 66.04) (width 0.5) (layer "F.Cu") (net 4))
 (segment (start 153.67 67.31) (end 152.4 66.04) (width 0.5) (layer "F.Cu") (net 4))
 (segment (start 166.37 84.6825) (end 168.615 84.6825) (width 0.5) (layer "F.Cu") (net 4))
 (segment (start 174.243 69.85) (end 179.07 69.85) (width 0.5) (layer "F.Cu") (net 4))
 (segment (start 180.34 71.12) (end 180.34 88.265) (width 0.5) (layer "F.Cu") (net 4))
 (segment (start 171.2225 89.535) (end 166.37 84.6825) (width 0.5) (layer "F.Cu") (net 4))
 (segment (start 174.243 69.85) (end 172.085 69.85) (width 0.5) (layer "F.Cu") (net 4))
 (segment (start 141.605 58.42) (end 149.225 66.04) (width 0.5) (layer "F.Cu") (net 4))
 (segment (start 166.37 84.6825) (end 165.84875 84.6825) (width 0.5) (layer "F.Cu") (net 4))
 (segment (start 149.225 66.04) (end 152.4 66.04) (width 0.5) (layer "F.Cu") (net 4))
 (segment (start 168.275 66.04) (end 152.4 66.04) (width 0.5) (layer "F.Cu") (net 4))
 (segment (start 165.84875 84.6825) (end 163.98625 82.82) (width 0.5) (layer "F.Cu") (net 4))
 (segment (start 157.4125 79.715) (end 157.1175 80.01) (width 0.5) (layer "F.Cu") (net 4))
 (segment (start 153.67 68.58) (end 153.67 67.31) (width 0.5) (layer "F.Cu") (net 4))
 (segment (start 141.605 55.49) (end 141.605 58.42) (width 0.5) (layer "F.Cu") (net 4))
 (segment (start 158.75 81.6425) (end 157.1175 80.01) (width 0.25) (layer "F.Cu") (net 4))
 (segment (start 180.34 88.265) (end 179.07 89.535) (width 0.5) (layer "F.Cu") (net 4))
 (segment (start 158.75 82.82) (end 162.56 82.82) (width 0.25) (layer "F.Cu") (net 4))
 (segment (start 157.4125 78.105) (end 157.4125 79.715) (width 0.5) (layer "F.Cu") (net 4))
 (segment (start 138.185 52.07) (end 141.605 55.49) (width 0.5) (layer "F.Cu") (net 4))
 (segment (start 158.75 82.82) (end 158.75 81.6425) (width 0.25) (layer "F.Cu") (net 4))
 (segment (start 174.243 77.47) (end 161.925 77.47) (width 0.5) (layer "F.Cu") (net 1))
 (segment (start 155.6875 77.3575) (end 155.6875 78.105) (width 0.5) (layer "F.Cu") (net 1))
 (segment (start 161.925 77.47) (end 160.655 76.2) (width 0.5) (layer "F.Cu") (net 1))
 (segment (start 146.05 83.185) (end 154.305 74.93) (width 0.5) (layer "F.Cu") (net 1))
 (segment (start 156.845 76.2) (end 155.6875 77.3575) (width 0.5) (layer "F.Cu") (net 1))
 (segment (start 154.35 81.6425) (end 155.9825 80.01) (width 0.25) (layer "F.Cu") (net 1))
 (segment (start 135.255 83.185) (end 145.415 83.185) (width 0.5) (layer "F.Cu") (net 1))
 (segment (start 154.94 74.93) (end 155.575 74.93) (width 0.5) (layer "F.Cu") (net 1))
 (segment (start 155.6875 78.105) (end 155.6875 79.715) (width 0.5) (layer "F.Cu") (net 1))
 (segment (start 148.59 74.93) (end 154.94 74.93) (width 0.5) (layer "F.Cu") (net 1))
 (segment (start 155.6875 79.715) (end 155.9825 80.01) (width 0.5) (layer "F.Cu") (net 1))
 (segment (start 154.305 74.93) (end 154.94 74.93) (width 0.5) (layer "F.Cu") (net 1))
 (segment (start 154.35 82.82) (end 154.35 81.6425) (width 0.25) (layer "F.Cu") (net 1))
 (segment (start 145.415 83.185) (end 146.05 83.185) (width 0.5) (layer "F.Cu") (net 1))
 (segment (start 160.655 76.2) (end 156.845 76.2) (width 0.5) (layer "F.Cu") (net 1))
 (segment (start 155.575 74.93) (end 156.845 76.2) (width 0.5) (layer "F.Cu") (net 1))
 (via (at 148.59 74.93) (size 0.8) (drill 0.4) (layers "F.Cu" "B.Cu") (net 1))
 (segment (start 148.59 68.58) (end 148.59 74.93) (width 0.5) (layer "B.Cu") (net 1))
 (segment (start 166.37 82.9575) (end 167.2325 82.9575) (width 0.5) (layer "F.Cu") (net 3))
 (segment (start 168.91 83.2525) (end 172.4055 83.2525) (width 0.5) (layer "F.Cu") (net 3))
 (segment (start 168.615 82.9575) (end 168.91 83.2525) (width 0.5) (layer "F.Cu") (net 3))
 (segment (start 172.4055 83.2525) (end 174.243 85.09) (width 0.5) (layer "F.Cu") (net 3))
 (segment (start 166.37 82.9575) (end 168.615 82.9575) (width 0.5) (layer "F.Cu") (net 3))
 (segment (start 167.2325 82.9575) (end 168.91 81.28) (width 0.5) (layer "F.Cu") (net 3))
 (via (at 168.91 81.28) (size 0.8) (drill 0.4) (layers "F.Cu" "B.Cu") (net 3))
 (segment (start 170.815 55.88) (end 163.83 48.895) (width 0.5) (layer "B.Cu") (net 3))
 (segment (start 137.16 48.895) (end 133.985 52.07) (width 0.5) (layer "B.Cu") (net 3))
 (segment (start 163.83 48.895) (end 137.16 48.895) (width 0.5) (layer "B.Cu") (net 3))
 (segment (start 170.815 79.375) (end 170.815 55.88) (width 0.5) (layer "B.Cu") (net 3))
 (segment (start 168.91 81.28) (end 170.815 79.375) (width 0.5) (layer "B.Cu") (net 3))
 (segment (start 158.75 84.82) (end 162.195 84.82) (width 0.25) (layer "F.Cu") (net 46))
 (segment (start 162.195 84.82) (end 163.195 83.82) (width 0.25) (layer "F.Cu") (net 46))
 (via (at 163.195 83.82) (size 0.8) (drill 0.4) (layers "F.Cu" "B.Cu") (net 46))
 (segment (start 144.78 60.96) (end 163.195 60.96) (width 0.25) (layer "B.Cu") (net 46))
 (segment (start 136.691 54.864) (end 138.684 54.864) (width 0.25) (layer "B.Cu") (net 46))
 (segment (start 169.545 67.31) (end 169.545 77.47) (width 0.25) (layer "B.Cu") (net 46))
 (segment (start 169.545 77.47) (end 163.195 83.82) (width 0.25) (layer "B.Cu") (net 46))
 (segment (start 133.985 57.57) (end 136.691 54.864) (width 0.25) (layer "B.Cu") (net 46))
 (segment (start 138.684 54.864) (end 144.78 60.96) (width 0.25) (layer "B.Cu") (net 46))
 (segment (start 163.195 60.96) (end 169.545 67.31) (width 0.25) (layer "B.Cu") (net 46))
 (segment (start 160.79 84.32) (end 161.29 83.82) (width 0.25) (layer "F.Cu") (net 47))
 (segment (start 158.75 84.32) (end 160.79 84.32) (width 0.25) (layer "F.Cu") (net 47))
 (via (at 161.29 83.82) (size 0.8) (drill 0.4) (layers "F.Cu" "B.Cu") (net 47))
 (segment (start 162.56 62.23) (end 168.275 67.945) (width 0.25) (layer "B.Cu") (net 47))
 (segment (start 142.845 62.23) (end 162.56 62.23) (width 0.25) (layer "B.Cu") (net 47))
 (segment (start 168.275 76.835) (end 161.29 83.82) (width 0.25) (layer "B.Cu") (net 47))
 (segment (start 168.275 67.945) (end 168.275 76.835) (width 0.25) (layer "B.Cu") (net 47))
 (segment (start 138.185 57.57) (end 142.845 62.23) (width 0.25) (layer "B.Cu") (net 47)))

